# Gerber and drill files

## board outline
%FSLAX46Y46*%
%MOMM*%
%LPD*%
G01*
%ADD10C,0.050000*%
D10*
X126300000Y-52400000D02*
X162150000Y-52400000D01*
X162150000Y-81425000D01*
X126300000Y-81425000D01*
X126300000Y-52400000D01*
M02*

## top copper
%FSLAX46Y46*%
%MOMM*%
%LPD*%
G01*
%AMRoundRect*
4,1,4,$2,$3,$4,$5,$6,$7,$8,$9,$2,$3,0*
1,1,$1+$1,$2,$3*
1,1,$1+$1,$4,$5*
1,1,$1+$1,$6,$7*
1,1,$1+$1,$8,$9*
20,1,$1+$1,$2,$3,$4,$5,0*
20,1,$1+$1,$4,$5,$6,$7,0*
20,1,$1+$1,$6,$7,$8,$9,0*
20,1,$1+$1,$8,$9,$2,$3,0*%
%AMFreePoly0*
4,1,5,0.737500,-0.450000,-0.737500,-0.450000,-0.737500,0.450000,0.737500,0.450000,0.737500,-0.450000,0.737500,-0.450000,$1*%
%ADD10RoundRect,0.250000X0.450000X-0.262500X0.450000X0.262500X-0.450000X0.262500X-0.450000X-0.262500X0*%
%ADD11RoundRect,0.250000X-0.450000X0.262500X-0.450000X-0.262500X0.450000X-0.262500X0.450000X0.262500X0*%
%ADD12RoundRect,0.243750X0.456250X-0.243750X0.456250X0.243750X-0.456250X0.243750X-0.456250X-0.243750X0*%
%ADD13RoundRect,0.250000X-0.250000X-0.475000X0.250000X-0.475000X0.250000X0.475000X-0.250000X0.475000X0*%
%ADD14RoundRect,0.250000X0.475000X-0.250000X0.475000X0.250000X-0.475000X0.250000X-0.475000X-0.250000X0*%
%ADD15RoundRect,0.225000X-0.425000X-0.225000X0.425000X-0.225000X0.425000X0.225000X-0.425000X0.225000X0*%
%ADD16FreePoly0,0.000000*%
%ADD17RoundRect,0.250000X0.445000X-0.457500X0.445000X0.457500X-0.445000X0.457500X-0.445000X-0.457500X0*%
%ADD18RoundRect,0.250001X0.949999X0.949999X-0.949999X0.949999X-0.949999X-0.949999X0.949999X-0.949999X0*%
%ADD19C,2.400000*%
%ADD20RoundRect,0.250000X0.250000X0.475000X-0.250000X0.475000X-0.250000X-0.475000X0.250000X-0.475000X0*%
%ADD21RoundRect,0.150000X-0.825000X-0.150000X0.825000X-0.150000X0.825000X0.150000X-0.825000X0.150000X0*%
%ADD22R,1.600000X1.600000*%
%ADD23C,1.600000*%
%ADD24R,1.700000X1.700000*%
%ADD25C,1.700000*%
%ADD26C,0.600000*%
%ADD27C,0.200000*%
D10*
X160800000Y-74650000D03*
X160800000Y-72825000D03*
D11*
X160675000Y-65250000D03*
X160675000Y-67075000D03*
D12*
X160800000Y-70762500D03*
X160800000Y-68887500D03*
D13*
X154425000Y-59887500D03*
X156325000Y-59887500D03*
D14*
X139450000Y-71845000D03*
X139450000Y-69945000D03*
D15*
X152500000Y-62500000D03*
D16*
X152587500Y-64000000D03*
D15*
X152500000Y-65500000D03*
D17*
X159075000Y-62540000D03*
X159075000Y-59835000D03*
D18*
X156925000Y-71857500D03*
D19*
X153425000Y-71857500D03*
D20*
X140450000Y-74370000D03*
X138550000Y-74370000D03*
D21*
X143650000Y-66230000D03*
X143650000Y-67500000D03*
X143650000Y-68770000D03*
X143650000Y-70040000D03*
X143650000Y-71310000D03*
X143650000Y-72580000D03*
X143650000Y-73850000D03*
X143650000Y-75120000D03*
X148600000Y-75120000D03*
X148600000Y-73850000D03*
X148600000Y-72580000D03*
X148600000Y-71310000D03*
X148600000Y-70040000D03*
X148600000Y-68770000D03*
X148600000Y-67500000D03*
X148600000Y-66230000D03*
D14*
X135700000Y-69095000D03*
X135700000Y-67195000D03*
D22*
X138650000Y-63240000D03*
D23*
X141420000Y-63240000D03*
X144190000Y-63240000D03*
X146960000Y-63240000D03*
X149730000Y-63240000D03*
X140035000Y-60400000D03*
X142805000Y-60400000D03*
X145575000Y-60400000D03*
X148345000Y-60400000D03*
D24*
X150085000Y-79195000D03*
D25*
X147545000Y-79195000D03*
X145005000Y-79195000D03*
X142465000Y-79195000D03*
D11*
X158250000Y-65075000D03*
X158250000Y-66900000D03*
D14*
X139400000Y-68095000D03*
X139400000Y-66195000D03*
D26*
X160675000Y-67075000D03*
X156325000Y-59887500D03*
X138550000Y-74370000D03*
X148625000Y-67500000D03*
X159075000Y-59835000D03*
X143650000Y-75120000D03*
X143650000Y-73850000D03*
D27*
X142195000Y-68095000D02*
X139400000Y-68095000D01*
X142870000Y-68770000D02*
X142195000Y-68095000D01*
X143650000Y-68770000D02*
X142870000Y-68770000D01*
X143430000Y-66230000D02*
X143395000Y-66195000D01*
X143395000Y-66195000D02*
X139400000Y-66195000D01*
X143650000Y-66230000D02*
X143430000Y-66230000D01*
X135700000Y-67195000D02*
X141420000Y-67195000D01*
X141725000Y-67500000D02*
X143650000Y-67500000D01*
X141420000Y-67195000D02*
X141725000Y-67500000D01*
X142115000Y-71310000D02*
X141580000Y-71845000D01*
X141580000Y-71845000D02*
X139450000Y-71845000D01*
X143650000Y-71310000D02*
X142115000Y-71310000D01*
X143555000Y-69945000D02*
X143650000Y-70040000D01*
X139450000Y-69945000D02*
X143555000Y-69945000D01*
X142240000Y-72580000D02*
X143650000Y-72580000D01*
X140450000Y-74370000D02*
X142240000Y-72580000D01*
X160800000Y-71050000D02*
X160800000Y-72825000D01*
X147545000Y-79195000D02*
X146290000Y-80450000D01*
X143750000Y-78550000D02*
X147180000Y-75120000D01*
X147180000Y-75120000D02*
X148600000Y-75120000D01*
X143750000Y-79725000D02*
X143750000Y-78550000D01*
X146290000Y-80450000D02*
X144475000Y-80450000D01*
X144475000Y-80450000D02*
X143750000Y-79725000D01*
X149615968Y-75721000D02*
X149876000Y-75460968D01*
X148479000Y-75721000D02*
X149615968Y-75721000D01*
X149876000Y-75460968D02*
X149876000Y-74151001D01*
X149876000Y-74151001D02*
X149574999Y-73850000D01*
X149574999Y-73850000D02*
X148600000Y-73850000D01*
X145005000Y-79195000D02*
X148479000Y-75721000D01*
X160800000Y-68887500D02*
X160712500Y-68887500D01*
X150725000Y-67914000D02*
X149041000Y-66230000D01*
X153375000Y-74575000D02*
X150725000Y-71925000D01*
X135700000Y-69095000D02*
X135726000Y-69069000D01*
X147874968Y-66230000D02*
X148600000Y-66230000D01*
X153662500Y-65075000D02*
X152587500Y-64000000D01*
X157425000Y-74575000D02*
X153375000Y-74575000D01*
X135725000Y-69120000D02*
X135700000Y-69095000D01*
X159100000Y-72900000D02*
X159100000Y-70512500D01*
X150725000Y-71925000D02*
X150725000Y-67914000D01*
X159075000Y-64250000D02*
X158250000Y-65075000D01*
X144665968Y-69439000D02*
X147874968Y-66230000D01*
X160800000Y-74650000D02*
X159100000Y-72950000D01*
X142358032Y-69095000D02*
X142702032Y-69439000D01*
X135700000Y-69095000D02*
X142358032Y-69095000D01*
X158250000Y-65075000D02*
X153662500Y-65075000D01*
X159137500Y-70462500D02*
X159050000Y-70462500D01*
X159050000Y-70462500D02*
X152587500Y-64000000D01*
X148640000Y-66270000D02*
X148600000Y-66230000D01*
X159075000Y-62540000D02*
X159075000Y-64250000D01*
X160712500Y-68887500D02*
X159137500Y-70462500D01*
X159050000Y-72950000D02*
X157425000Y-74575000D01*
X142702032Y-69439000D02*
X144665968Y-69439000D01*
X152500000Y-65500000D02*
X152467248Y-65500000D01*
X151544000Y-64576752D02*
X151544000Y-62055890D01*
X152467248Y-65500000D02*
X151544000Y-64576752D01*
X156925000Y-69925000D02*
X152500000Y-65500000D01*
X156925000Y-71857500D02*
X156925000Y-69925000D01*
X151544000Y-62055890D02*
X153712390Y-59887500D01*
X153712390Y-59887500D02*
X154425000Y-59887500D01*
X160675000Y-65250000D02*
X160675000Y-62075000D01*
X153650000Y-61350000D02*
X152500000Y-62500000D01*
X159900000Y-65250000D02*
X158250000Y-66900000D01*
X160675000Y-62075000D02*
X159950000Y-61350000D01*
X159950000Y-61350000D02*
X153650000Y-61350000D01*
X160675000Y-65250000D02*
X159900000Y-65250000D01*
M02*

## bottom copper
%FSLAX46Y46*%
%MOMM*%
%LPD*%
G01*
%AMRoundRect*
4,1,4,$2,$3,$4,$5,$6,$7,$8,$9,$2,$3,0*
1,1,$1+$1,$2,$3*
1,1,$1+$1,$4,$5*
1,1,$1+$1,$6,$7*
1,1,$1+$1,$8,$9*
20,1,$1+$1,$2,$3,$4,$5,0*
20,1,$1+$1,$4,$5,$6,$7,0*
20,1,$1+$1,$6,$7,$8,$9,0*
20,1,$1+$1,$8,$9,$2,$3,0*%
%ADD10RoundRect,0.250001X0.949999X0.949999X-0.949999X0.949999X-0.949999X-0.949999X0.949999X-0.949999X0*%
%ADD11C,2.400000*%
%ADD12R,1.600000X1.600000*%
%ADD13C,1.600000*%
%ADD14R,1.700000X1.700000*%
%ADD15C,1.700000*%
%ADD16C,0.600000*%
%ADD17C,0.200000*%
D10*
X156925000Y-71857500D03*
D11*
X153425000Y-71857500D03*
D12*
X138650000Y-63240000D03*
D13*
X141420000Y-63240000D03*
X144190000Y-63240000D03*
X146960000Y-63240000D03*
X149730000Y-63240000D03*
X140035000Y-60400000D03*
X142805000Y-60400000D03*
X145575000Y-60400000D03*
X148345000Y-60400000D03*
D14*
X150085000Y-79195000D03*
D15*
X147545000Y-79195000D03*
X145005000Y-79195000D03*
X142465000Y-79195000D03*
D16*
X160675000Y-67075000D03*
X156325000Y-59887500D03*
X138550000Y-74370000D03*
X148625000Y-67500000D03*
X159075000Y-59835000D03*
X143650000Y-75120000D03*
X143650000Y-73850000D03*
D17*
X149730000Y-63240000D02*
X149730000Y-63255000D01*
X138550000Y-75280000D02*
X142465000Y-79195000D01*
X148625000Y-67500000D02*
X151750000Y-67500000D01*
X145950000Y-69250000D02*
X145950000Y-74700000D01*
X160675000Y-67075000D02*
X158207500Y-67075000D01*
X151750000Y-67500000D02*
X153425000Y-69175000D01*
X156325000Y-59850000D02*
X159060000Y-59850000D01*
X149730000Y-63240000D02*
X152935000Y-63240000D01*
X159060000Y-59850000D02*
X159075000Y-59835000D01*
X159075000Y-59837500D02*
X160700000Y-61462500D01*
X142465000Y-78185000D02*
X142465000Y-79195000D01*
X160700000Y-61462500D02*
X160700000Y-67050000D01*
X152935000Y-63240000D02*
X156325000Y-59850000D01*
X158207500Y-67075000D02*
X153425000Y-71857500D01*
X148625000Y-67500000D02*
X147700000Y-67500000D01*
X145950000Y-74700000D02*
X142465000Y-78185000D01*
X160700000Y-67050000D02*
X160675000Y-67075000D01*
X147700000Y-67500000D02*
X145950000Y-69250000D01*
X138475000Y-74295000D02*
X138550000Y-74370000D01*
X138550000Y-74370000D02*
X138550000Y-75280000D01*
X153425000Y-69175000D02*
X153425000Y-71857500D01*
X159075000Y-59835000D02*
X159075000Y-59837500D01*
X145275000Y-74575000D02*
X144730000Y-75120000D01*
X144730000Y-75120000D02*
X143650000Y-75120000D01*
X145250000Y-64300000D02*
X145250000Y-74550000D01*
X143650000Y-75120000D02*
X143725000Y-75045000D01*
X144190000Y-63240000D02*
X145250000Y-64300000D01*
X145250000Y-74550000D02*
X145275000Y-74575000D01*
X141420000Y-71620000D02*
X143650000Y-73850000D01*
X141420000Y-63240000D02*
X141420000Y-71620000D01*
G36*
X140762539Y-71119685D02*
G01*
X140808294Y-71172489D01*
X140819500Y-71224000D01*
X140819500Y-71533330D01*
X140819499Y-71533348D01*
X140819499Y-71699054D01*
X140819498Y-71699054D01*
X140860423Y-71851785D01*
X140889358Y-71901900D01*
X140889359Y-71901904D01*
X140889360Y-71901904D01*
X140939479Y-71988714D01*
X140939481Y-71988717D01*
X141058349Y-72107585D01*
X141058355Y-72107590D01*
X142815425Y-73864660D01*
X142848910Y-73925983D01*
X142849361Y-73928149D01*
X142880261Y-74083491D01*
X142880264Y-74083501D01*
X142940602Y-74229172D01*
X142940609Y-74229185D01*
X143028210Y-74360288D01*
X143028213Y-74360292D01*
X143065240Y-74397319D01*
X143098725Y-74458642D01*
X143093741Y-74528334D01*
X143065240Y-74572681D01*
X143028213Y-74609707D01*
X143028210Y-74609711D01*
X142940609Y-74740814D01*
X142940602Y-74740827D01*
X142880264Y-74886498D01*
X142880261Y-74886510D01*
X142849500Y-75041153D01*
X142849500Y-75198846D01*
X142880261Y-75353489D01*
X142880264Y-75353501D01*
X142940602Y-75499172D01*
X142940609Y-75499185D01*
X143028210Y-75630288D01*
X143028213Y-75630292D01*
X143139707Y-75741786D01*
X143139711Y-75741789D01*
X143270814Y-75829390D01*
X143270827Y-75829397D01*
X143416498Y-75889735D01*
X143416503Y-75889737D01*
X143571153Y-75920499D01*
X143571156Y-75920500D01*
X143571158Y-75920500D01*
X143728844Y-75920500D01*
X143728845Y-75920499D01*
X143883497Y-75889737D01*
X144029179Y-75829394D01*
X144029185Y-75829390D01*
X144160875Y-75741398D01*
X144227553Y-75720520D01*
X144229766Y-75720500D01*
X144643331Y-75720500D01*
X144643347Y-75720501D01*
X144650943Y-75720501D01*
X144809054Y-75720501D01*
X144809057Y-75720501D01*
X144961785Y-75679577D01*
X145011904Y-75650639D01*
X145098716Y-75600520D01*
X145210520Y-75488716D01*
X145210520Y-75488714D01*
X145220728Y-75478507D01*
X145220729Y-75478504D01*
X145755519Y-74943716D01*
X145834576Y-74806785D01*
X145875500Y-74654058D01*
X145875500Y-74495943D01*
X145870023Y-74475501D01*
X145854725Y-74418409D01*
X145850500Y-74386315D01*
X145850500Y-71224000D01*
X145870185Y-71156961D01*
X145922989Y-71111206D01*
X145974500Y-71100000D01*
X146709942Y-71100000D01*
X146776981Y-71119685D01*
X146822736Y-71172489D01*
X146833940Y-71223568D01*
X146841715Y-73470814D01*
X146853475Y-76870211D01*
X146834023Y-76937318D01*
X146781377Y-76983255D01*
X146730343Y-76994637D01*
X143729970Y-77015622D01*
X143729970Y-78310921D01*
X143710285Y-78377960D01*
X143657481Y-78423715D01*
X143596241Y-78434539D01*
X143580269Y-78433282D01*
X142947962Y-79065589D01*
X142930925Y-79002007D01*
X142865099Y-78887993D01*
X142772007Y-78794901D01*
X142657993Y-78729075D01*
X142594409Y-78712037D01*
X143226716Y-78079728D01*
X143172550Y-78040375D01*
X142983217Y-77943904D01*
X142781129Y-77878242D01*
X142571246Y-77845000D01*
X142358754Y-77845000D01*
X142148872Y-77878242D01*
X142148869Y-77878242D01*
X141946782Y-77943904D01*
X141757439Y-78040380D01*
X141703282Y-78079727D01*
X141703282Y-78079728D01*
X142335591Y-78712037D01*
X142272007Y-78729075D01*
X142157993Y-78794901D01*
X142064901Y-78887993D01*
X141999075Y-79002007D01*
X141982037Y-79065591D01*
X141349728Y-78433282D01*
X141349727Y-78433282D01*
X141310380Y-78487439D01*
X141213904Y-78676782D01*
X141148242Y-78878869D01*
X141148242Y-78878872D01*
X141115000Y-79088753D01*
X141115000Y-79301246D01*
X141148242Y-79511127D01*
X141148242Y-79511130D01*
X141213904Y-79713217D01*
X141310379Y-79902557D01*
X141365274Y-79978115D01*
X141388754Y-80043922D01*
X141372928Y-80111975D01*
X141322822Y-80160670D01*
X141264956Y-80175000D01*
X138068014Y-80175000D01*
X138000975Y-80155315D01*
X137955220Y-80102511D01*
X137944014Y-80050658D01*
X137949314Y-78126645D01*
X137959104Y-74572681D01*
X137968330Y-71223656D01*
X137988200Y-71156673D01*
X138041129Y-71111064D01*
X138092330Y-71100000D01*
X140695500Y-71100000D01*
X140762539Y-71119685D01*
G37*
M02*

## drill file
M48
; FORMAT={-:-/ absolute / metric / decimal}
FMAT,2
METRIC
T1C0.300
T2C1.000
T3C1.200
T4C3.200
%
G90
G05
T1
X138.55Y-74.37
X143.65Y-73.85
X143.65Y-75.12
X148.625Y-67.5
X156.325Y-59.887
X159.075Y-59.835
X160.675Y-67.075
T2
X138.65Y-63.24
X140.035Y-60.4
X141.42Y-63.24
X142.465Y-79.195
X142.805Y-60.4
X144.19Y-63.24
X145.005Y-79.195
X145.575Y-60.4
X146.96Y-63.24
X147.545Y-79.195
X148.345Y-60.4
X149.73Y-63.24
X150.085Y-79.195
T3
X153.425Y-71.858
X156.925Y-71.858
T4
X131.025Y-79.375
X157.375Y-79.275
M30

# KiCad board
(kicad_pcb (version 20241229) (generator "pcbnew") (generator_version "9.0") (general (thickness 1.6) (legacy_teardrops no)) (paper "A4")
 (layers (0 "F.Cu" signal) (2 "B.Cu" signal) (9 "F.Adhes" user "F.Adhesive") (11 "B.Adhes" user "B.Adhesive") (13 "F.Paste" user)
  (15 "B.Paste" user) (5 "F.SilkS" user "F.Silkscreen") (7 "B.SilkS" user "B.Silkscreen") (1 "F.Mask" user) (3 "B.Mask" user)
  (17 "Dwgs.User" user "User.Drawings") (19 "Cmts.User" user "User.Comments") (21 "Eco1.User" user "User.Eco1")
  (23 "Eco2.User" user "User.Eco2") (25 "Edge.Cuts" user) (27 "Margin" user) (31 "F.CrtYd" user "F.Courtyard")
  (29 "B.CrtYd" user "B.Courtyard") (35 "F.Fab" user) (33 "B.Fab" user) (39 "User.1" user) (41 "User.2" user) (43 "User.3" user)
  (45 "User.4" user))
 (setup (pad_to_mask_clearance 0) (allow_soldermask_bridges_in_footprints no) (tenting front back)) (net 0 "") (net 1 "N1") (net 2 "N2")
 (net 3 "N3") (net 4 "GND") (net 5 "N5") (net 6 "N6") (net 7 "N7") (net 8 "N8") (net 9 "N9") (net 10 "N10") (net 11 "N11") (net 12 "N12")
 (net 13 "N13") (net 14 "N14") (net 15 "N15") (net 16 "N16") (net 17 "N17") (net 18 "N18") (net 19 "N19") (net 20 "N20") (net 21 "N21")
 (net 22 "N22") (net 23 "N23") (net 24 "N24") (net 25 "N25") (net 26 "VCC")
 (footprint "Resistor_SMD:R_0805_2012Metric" (layer "F.Cu") (at 160.8 73.7375 90)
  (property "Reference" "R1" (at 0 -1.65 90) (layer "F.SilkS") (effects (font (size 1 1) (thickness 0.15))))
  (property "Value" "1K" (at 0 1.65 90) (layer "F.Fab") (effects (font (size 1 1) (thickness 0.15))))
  (pad "1" smd roundrect (at -0.9125 0 90) (size 1.025 1.4) (layers "F.Cu" "F.Mask" "F.Paste") (roundrect_rratio 0.243902) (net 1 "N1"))
  (pad "2" smd roundrect (at 0.9125 0 90) (size 1.025 1.4) (layers "F.Cu" "F.Mask" "F.Paste") (roundrect_rratio 0.243902) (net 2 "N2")))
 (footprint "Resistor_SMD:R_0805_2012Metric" (layer "F.Cu") (at 160.675 66.1625 -90)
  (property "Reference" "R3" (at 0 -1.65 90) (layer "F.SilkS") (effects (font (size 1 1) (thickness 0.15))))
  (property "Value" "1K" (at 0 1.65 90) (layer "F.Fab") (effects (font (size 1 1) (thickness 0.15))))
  (pad "1" smd roundrect (at -0.9125 0 270) (size 1.025 1.4) (layers "F.Cu" "F.Mask" "F.Paste") (roundrect_rratio 0.243902) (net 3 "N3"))
  (pad "2" smd roundrect (at 0.9125 0 270) (size 1.025 1.4) (layers "F.Cu" "F.Mask" "F.Paste") (roundrect_rratio 0.243902) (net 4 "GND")))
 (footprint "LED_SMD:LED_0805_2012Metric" (layer "F.Cu") (at 160.8 69.825 90)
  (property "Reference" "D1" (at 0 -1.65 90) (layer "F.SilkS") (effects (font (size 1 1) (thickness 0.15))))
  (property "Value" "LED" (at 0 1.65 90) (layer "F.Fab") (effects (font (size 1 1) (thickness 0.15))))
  (pad "1" smd roundrect (at -0.9375 0 90) (size 0.975 1.4) (layers "F.Cu" "F.Mask" "F.Paste") (roundrect_rratio 0.25) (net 2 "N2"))
  (pad "2" smd roundrect (at 0.9375 0 90) (size 0.975 1.4) (layers "F.Cu" "F.Mask" "F.Paste") (roundrect_rratio 0.25) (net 1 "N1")))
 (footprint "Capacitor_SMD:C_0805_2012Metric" (layer "F.Cu") (at 155.375 59.8875)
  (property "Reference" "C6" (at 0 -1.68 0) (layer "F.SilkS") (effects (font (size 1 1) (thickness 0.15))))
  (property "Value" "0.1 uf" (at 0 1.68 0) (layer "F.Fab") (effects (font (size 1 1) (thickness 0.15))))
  (pad "1" smd roundrect (at -0.95 0) (size 1 1.45) (layers "F.Cu" "F.Mask" "F.Paste") (roundrect_rratio 0.25) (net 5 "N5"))
  (pad "2" smd roundrect (at 0.95 0) (size 1 1.45) (layers "F.Cu" "F.Mask" "F.Paste") (roundrect_rratio 0.25) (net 4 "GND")))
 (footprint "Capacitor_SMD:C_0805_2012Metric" (layer "F.Cu") (at 139.45 70.895 90)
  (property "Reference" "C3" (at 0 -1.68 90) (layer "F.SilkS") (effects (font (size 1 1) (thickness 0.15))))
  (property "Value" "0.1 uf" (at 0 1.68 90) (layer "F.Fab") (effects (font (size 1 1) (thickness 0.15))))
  (pad "1" smd roundrect (at -0.95 0 90) (size 1 1.45) (layers "F.Cu" "F.Mask" "F.Paste") (roundrect_rratio 0.25) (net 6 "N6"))
  (pad "2" smd roundrect (at 0.95 0 90) (size 1 1.45) (layers "F.Cu" "F.Mask" "F.Paste") (roundrect_rratio 0.25) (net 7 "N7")))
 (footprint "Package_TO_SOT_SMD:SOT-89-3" (layer "F.Cu") (at 154.45 64)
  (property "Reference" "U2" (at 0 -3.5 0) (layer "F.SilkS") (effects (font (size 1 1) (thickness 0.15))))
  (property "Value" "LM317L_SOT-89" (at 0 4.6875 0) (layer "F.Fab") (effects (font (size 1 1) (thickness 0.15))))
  (pad "1" smd roundrect (at -1.95 -1.5) (size 1.3 0.9) (layers "F.Cu" "F.Mask" "F.Paste") (roundrect_rratio 0.25) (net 3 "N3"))
  (pad "2" smd custom (at -1.8625 0) (size 1.475 0.9) (layers "F.Cu" "F.Mask" "F.Paste") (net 1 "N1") (zone_connect 2)
   (thermal_bridge_angle 45) (options (clearance outline) (anchor rect)) (primitives))
  (pad "3" smd roundrect (at -1.95 1.5) (size 1.3 0.9) (layers "F.Cu" "F.Mask" "F.Paste") (roundrect_rratio 0.25) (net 5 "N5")))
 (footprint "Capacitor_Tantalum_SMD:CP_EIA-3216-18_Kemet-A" (layer "F.Cu") (at 159.075 61.1875 90)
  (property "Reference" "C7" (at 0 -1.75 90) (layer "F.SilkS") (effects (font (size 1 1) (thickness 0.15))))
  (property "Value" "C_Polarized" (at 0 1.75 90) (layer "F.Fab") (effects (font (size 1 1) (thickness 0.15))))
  (pad "1" smd roundrect (at -1.3525 0 90) (size 1.415 1.39) (layers "F.Cu" "F.Mask" "F.Paste") (roundrect_rratio 0.179856) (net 1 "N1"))
  (pad "2" smd roundrect (at 1.3525 0 90) (size 1.415 1.39) (layers "F.Cu" "F.Mask" "F.Paste") (roundrect_rratio 0.179856) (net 4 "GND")))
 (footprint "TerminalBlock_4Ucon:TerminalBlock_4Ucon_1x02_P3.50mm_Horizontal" (layer "F.Cu") (at 156.925 71.8575 180)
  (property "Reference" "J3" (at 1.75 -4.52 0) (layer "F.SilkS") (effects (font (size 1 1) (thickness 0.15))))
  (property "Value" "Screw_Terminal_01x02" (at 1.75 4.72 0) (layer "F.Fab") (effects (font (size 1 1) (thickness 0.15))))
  (pad "1" thru_hole roundrect (at 0 0 180) (size 2.4 2.4) (drill 1.2) (layers "*.Cu" "*.Mask") (remove_unused_layers no)
   (roundrect_rratio 0.104167) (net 5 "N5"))
  (pad "2" thru_hole circle (at 3.5 0 180) (size 2.4 2.4) (drill 1.2) (layers "*.Cu" "*.Mask") (remove_unused_layers no) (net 4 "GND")))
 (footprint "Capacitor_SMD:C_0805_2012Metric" (layer "F.Cu") (at 139.5 74.37 180)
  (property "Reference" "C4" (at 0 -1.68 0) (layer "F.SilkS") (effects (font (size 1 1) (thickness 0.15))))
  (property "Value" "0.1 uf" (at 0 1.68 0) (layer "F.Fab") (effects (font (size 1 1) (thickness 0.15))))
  (pad "1" smd roundrect (at -0.95 0 180) (size 1 1.45) (layers "F.Cu" "F.Mask" "F.Paste") (roundrect_rratio 0.25) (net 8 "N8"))
  (pad "2" smd roundrect (at 0.95 0 180) (size 1 1.45) (layers "F.Cu" "F.Mask" "F.Paste") (roundrect_rratio 0.25) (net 4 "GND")))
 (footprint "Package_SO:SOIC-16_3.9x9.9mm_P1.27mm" (layer "F.Cu") (at 146.125 70.675)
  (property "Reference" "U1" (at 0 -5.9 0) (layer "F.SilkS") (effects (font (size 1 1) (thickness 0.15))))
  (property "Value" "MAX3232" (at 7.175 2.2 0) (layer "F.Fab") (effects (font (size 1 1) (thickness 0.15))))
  (pad "1" smd roundrect (at -2.475 -4.445) (size 1.95 0.6) (layers "F.Cu" "F.Mask" "F.Paste") (roundrect_rratio 0.25) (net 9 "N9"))
  (pad "2" smd roundrect (at -2.475 -3.175) (size 1.95 0.6) (layers "F.Cu" "F.Mask" "F.Paste") (roundrect_rratio 0.25) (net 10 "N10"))
  (pad "3" smd roundrect (at -2.475 -1.905) (size 1.95 0.6) (layers "F.Cu" "F.Mask" "F.Paste") (roundrect_rratio 0.25) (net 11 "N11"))
  (pad "4" smd roundrect (at -2.475 -0.635) (size 1.95 0.6) (layers "F.Cu" "F.Mask" "F.Paste") (roundrect_rratio 0.25) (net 7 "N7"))
  (pad "5" smd roundrect (at -2.475 0.635) (size 1.95 0.6) (layers "F.Cu" "F.Mask" "F.Paste") (roundrect_rratio 0.25) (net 6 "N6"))
  (pad "6" smd roundrect (at -2.475 1.905) (size 1.95 0.6) (layers "F.Cu" "F.Mask" "F.Paste") (roundrect_rratio 0.25) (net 8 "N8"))
  (pad "7" smd roundrect (at -2.475 3.175) (size 1.95 0.6) (layers "F.Cu" "F.Mask" "F.Paste") (roundrect_rratio 0.25) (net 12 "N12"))
  (pad "8" smd roundrect (at -2.475 4.445) (size 1.95 0.6) (layers "F.Cu" "F.Mask" "F.Paste") (roundrect_rratio 0.25) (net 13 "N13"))
  (pad "9" smd roundrect (at 2.475 4.445) (size 1.95 0.6) (layers "F.Cu" "F.Mask" "F.Paste") (roundrect_rratio 0.25) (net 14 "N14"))
  (pad "10" smd roundrect (at 2.475 3.175) (size 1.95 0.6) (layers "F.Cu" "F.Mask" "F.Paste") (roundrect_rratio 0.25) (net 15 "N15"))
  (pad "11" smd roundrect (at 2.475 1.905) (size 1.95 0.6) (layers "F.Cu" "F.Mask" "F.Paste") (roundrect_rratio 0.25) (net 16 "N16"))
  (pad "12" smd roundrect (at 2.475 0.635) (size 1.95 0.6) (layers "F.Cu" "F.Mask" "F.Paste") (roundrect_rratio 0.25) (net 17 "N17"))
  (pad "13" smd roundrect (at 2.475 -0.635) (size 1.95 0.6) (layers "F.Cu" "F.Mask" "F.Paste") (roundrect_rratio 0.25) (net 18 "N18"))
  (pad "14" smd roundrect (at 2.475 -1.905) (size 1.95 0.6) (layers "F.Cu" "F.Mask" "F.Paste") (roundrect_rratio 0.25) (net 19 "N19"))
  (pad "15" smd roundrect (at 2.475 -3.175) (size 1.95 0.6) (layers "F.Cu" "F.Mask" "F.Paste") (roundrect_rratio 0.25) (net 4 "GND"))
  (pad "16" smd roundrect (at 2.475 -4.445) (size 1.95 0.6) (layers "F.Cu" "F.Mask" "F.Paste") (roundrect_rratio 0.25) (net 1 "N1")))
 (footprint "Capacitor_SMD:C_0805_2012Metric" (layer "F.Cu") (at 135.7 68.145 90)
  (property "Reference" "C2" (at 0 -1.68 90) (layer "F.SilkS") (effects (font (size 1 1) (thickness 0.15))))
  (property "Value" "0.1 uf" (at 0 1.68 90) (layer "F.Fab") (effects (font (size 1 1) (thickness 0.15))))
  (pad "1" smd roundrect (at -0.95 0 90) (size 1 1.45) (layers "F.Cu" "F.Mask" "F.Paste") (roundrect_rratio 0.25) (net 1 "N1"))
  (pad "2" smd roundrect (at 0.95 0 90) (size 1 1.45) (layers "F.Cu" "F.Mask" "F.Paste") (roundrect_rratio 0.25) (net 10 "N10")))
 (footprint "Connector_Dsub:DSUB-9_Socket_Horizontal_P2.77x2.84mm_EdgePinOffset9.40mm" (layer "F.Cu") (at 138.65 63.24 180)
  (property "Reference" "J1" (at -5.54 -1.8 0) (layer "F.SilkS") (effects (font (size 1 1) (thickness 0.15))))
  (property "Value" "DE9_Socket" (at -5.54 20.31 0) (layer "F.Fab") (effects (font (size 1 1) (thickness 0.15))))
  (pad "1" thru_hole rect (at 0 0 180) (size 1.6 1.6) (drill 1) (layers "*.Cu" "*.Mask") (remove_unused_layers no) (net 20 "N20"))
  (pad "2" thru_hole circle (at -2.77 0 180) (size 1.6 1.6) (drill 1) (layers "*.Cu" "*.Mask") (remove_unused_layers no) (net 12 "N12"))
  (pad "3" thru_hole circle (at -5.54 0 180) (size 1.6 1.6) (drill 1) (layers "*.Cu" "*.Mask") (remove_unused_layers no) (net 13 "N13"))
  (pad "4" thru_hole circle (at -8.31 0 180) (size 1.6 1.6) (drill 1) (layers "*.Cu" "*.Mask") (remove_unused_layers no) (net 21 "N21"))
  (pad "5" thru_hole circle (at -11.08 0 180) (size 1.6 1.6) (drill 1) (layers "*.Cu" "*.Mask") (remove_unused_layers no) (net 4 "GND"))
  (pad "6" thru_hole circle (at -1.385 2.84 180) (size 1.6 1.6) (drill 1) (layers "*.Cu" "*.Mask") (remove_unused_layers no) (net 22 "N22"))
  (pad "7" thru_hole circle (at -4.155 2.84 180) (size 1.6 1.6) (drill 1) (layers "*.Cu" "*.Mask") (remove_unused_layers no) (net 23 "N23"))
  (pad "8" thru_hole circle (at -6.925 2.84 180) (size 1.6 1.6) (drill 1) (layers "*.Cu" "*.Mask") (remove_unused_layers no) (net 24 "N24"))
  (pad "9" thru_hole circle (at -9.695 2.84 180) (size 1.6 1.6) (drill 1) (layers "*.Cu" "*.Mask") (remove_unused_layers no) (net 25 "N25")))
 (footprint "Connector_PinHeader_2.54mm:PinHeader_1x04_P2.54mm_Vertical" (layer "F.Cu") (at 150.085 79.195 -90)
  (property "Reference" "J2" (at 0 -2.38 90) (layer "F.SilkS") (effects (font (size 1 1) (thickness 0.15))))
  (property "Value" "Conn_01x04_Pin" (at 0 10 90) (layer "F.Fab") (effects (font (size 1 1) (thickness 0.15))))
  (pad "1" thru_hole rect (at 0 0 270) (size 1.7 1.7) (drill 1) (layers "*.Cu" "*.Mask") (remove_unused_layers no) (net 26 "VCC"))
  (pad "2" thru_hole circle (at 0 2.54 270) (size 1.7 1.7) (drill 1) (layers "*.Cu" "*.Mask") (remove_unused_layers no) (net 14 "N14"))
  (pad "3" thru_hole circle (at 0 5.08 270) (size 1.7 1.7) (drill 1) (layers "*.Cu" "*.Mask") (remove_unused_layers no) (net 15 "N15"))
  (pad "4" thru_hole circle (at 0 7.62 270) (size 1.7 1.7) (drill 1) (layers "*.Cu" "*.Mask") (remove_unused_layers no) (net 4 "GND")))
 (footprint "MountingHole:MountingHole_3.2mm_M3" (layer "F.Cu") (at 157.375 79.275)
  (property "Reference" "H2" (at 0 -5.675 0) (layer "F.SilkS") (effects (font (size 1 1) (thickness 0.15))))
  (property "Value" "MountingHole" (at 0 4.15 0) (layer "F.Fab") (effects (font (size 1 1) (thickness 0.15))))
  (pad "" np_thru_hole circle (at 0 0) (size 3.2 3.2) (drill 3.2) (layers "*.Cu" "*.Mask")))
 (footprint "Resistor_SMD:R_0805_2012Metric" (layer "F.Cu") (at 158.25 65.9875 -90)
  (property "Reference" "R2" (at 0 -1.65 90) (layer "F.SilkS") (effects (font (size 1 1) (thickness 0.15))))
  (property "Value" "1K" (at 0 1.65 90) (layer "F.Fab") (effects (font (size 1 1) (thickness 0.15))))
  (pad "1" smd roundrect (at -0.9125 0 270) (size 1.025 1.4) (layers "F.Cu" "F.Mask" "F.Paste") (roundrect_rratio 0.243902) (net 1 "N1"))
  (pad "2" smd roundrect (at 0.9125 0 270) (size 1.025 1.4) (layers "F.Cu" "F.Mask" "F.Paste") (roundrect_rratio 0.243902) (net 3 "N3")))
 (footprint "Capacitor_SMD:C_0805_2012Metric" (layer "F.Cu") (at 139.4 67.145 90)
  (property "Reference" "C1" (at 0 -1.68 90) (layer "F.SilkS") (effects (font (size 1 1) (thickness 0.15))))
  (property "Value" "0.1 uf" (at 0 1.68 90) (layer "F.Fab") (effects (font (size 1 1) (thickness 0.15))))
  (pad "1" smd roundrect (at -0.95 0 90) (size 1 1.45) (layers "F.Cu" "F.Mask" "F.Paste") (roundrect_rratio 0.25) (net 11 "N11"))
  (pad "2" smd roundrect (at 0.95 0 90) (size 1 1.45) (layers "F.Cu" "F.Mask" "F.Paste") (roundrect_rratio 0.25) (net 9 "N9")))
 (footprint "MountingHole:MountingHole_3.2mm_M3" (layer "F.Cu") (at 131.025 79.375)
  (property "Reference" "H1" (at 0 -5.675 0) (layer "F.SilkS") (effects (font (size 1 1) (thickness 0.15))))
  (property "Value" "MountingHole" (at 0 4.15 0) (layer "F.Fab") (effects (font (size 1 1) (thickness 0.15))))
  (pad "" np_thru_hole circle (at 0 0) (size 3.2 3.2) (drill 3.2) (layers "*.Cu" "*.Mask")))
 (gr_rect (start 126.3 52.4) (end 162.15 81.425) (stroke (width 0.05) (type solid)) (fill no) (layer "Edge.Cuts"))
 (segment (start 142.195 68.095) (end 139.4 68.095) (width 0.2) (layer "F.Cu") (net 11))
 (segment (start 142.87 68.77) (end 142.195 68.095) (width 0.2) (layer "F.Cu") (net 11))
 (segment (start 143.65 68.77) (end 142.87 68.77) (width 0.2) (layer "F.Cu") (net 11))
 (segment (start 143.43 66.23) (end 143.395 66.195) (width 0.2) (layer "F.Cu") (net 9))
 (segment (start 143.395 66.195) (end 139.4 66.195) (width 0.2) (layer "F.Cu") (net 9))
 (segment (start 143.65 66.23) (end 143.43 66.23) (width 0.2) (layer "F.Cu") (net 9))
 (segment (start 135.7 67.195) (end 141.42 67.195) (width 0.2) (layer "F.Cu") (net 10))
 (segment (start 141.725 67.5) (end 143.65 67.5) (width 0.2) (layer "F.Cu") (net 10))
 (segment (start 141.42 67.195) (end 141.725 67.5) (width 0.2) (layer "F.Cu") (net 10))
 (segment (start 142.115 71.31) (end 141.58 71.845) (width 0.2) (layer "F.Cu") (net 6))
 (segment (start 141.58 71.845) (end 139.45 71.845) (width 0.2) (layer "F.Cu") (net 6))
 (segment (start 143.65 71.31) (end 142.115 71.31) (width 0.2) (layer "F.Cu") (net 6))
 (segment (start 143.555 69.945) (end 143.65 70.04) (width 0.2) (layer "F.Cu") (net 7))
 (segment (start 139.45 69.945) (end 143.555 69.945) (width 0.2) (layer "F.Cu") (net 7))
 (via (at 160.675 67.075) (size 0.6) (drill 0.3) (layers "F.Cu" "B.Cu") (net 4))
 (via (at 156.325 59.8875) (size 0.6) (drill 0.3) (layers "F.Cu" "B.Cu") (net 4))
 (via (at 138.55 74.37) (size 0.6) (drill 0.3) (layers "F.Cu" "B.Cu") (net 4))
 (via (at 148.625 67.5) (size 0.6) (drill 0.3) (layers "F.Cu" "B.Cu") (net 4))
 (via (at 159.075 59.835) (size 0.6) (drill 0.3) (layers "F.Cu" "B.Cu") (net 4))
 (segment (start 149.73 63.24) (end 149.73 63.255) (width 0.2) (layer "B.Cu") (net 4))
 (segment (start 138.55 75.28) (end 142.465 79.195) (width 0.2) (layer "B.Cu") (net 4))
 (segment (start 148.625 67.5) (end 151.75 67.5) (width 0.2) (layer "B.Cu") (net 4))
 (segment (start 145.95 69.25) (end 145.95 74.7) (width 0.2) (layer "B.Cu") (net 4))
 (segment (start 160.675 67.075) (end 158.2075 67.075) (width 0.2) (layer "B.Cu") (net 4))
 (segment (start 151.75 67.5) (end 153.425 69.175) (width 0.2) (layer "B.Cu") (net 4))
 (segment (start 156.325 59.85) (end 159.06 59.85) (width 0.2) (layer "B.Cu") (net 4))
 (segment (start 149.73 63.24) (end 152.935 63.24) (width 0.2) (layer "B.Cu") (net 4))
 (segment (start 159.06 59.85) (end 159.075 59.835) (width 0.2) (layer "B.Cu") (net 4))
 (segment (start 159.075 59.8375) (end 160.7 61.4625) (width 0.2) (layer "B.Cu") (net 4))
 (segment (start 142.465 78.185) (end 142.465 79.195) (width 0.2) (layer "B.Cu") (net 4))
 (segment (start 160.7 61.4625) (end 160.7 67.05) (width 0.2) (layer "B.Cu") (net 4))
 (segment (start 152.935 63.24) (end 156.325 59.85) (width 0.2) (layer "B.Cu") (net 4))
 (segment (start 158.2075 67.075) (end 153.425 71.8575) (width 0.2) (layer "B.Cu") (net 4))
 (segment (start 148.625 67.5) (end 147.7 67.5) (width 0.2) (layer "B.Cu") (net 4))
 (segment (start 145.95 74.7) (end 142.465 78.185) (width 0.2) (layer "B.Cu") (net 4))
 (segment (start 160.7 67.05) (end 160.675 67.075) (width 0.2) (layer "B.Cu") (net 4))
 (segment (start 147.7 67.5) (end 145.95 69.25) (width 0.2) (layer "B.Cu") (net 4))
 (segment (start 138.475 74.295) (end 138.55 74.37) (width 0.2) (layer "B.Cu") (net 4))
 (segment (start 138.55 74.37) (end 138.55 75.28) (width 0.2) (layer "B.Cu") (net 4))
 (segment (start 153.425 69.175) (end 153.425 71.8575) (width 0.2) (layer "B.Cu") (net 4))
 (segment (start 159.075 59.835) (end 159.075 59.8375) (width 0.2) (layer "B.Cu") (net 4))
 (segment (start 142.24 72.58) (end 143.65 72.58) (width 0.2) (layer "F.Cu") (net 8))
 (segment (start 140.45 74.37) (end 142.24 72.58) (width 0.2) (layer "F.Cu") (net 8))
 (segment (start 160.8 71.05) (end 160.8 72.825) (width 0.2) (layer "F.Cu") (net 2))
 (via (at 143.65 75.12) (size 0.6) (drill 0.3) (layers "F.Cu" "B.Cu") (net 13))
 (segment (start 145.275 74.575) (end 144.73 75.12) (width 0.2) (layer "B.Cu") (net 13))
 (segment (start 144.73 75.12) (end 143.65 75.12) (width 0.2) (layer "B.Cu") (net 13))
 (segment (start 145.25 64.3) (end 145.25 74.55) (width 0.2) (layer "B.Cu") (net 13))
 (segment (start 143.65 75.12) (end 143.725 75.045) (width 0.2) (layer "B.Cu") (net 13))
 (segment (start 144.19 63.24) (end 145.25 64.3) (width 0.2) (layer "B.Cu") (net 13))
 (segment (start 145.25 74.55) (end 145.275 74.575) (width 0.2) (layer "B.Cu") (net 13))
 (via (at 143.65 73.85) (size 0.6) (drill 0.3) (layers "F.Cu" "B.Cu") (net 12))
 (segment (start 141.42 71.62) (end 143.65 73.85) (width 0.2) (layer "B.Cu") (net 12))
 (segment (start 141.42 63.24) (end 141.42 71.62) (width 0.2) (layer "B.Cu") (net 12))
 (segment (start 147.545 79.195) (end 146.29 80.45) (width 0.2) (layer "F.Cu") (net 14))
 (segment (start 143.75 78.55) (end 147.18 75.12) (width 0.2) (layer "F.Cu") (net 14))
 (segment (start 147.18 75.12) (end 148.6 75.12) (width 0.2) (layer "F.Cu") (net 14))
 (segment (start 143.75 79.725) (end 143.75 78.55) (width 0.2) (layer "F.Cu") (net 14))
 (segment (start 146.29 80.45) (end 144.475 80.45) (width 0.2) (layer "F.Cu") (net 14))
 (segment (start 144.475 80.45) (end 143.75 79.725) (width 0.2) (layer "F.Cu") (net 14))
 (segment (start 149.615968 75.721) (end 149.876 75.460968) (width 0.2) (layer "F.Cu") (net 15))
 (segment (start 148.479 75.721) (end 149.615968 75.721) (width 0.2) (layer "F.Cu") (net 15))
 (segment (start 149.876 75.460968) (end 149.876 74.151001) (width 0.2) (layer "F.Cu") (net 15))
 (segment (start 149.876 74.151001) (end 149.574999 73.85) (width 0.2) (layer "F.Cu") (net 15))
 (segment (start 149.574999 73.85) (end 148.6 73.85) (width 0.2) (layer "F.Cu") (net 15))
 (segment (start 145.005 79.195) (end 148.479 75.721) (width 0.2) (layer "F.Cu") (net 15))
 (segment (start 160.8 68.8875) (end 160.7125 68.8875) (width 0.2) (layer "F.Cu") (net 1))
 (segment (start 150.725 67.914) (end 149.041 66.23) (width 0.2) (layer "F.Cu") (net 1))
 (segment (start 153.375 74.575) (end 150.725 71.925) (width 0.2) (layer "F.Cu") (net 1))
 (segment (start 135.7 69.095) (end 135.726 69.069) (width 0.2) (layer "F.Cu") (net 1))
 (segment (start 147.874968 66.23) (end 148.6 66.23) (width 0.2) (layer "F.Cu") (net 1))
 (segment (start 153.6625 65.075) (end 152.5875 64) (width 0.2) (layer "F.Cu") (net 1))
 (segment (start 157.425 74.575) (end 153.375 74.575) (width 0.2) (layer "F.Cu") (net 1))
 (segment (start 135.725 69.12) (end 135.7 69.095) (width 0.2) (layer "F.Cu") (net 1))
 (segment (start 159.1 72.9) (end 159.1 70.5125) (width 0.2) (layer "F.Cu") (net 1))
 (segment (start 150.725 71.925) (end 150.725 67.914) (width 0.2) (layer "F.Cu") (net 1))
 (segment (start 159.075 64.25) (end 158.25 65.075) (width 0.2) (layer "F.Cu") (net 1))
 (segment (start 144.665968 69.439) (end 147.874968 66.23) (width 0.2) (layer "F.Cu") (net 1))
 (segment (start 160.8 74.65) (end 159.1 72.95) (width 0.2) (layer "F.Cu") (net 1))
 (segment (start 142.358032 69.095) (end 142.702032 69.439) (width 0.2) (layer "F.Cu") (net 1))
 (segment (start 135.7 69.095) (end 142.358032 69.095) (width 0.2) (layer "F.Cu") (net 1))
 (segment (start 158.25 65.075) (end 153.6625 65.075) (width 0.2) (layer "F.Cu") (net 1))
 (segment (start 159.1375 70.4625) (end 159.05 70.4625) (width 0.2) (layer "F.Cu") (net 1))
 (segment (start 159.05 70.4625) (end 152.5875 64) (width 0.2) (layer "F.Cu") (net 1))
 (segment (start 148.64 66.27) (end 148.6 66.23) (width 0.2) (layer "F.Cu") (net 1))
 (segment (start 159.075 62.54) (end 159.075 64.25) (width 0.2) (layer "F.Cu") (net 1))
 (segment (start 160.7125 68.8875) (end 159.1375 70.4625) (width 0.2) (layer "F.Cu") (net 1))
 (segment (start 159.05 72.95) (end 157.425 74.575) (width 0.2) (layer "F.Cu") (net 1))
 (segment (start 142.702032 69.439) (end 144.665968 69.439) (width 0.2) (layer "F.Cu") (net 1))
 (segment (start 152.5 65.5) (end 152.467248 65.5) (width 0.2) (layer "F.Cu") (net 5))
 (segment (start 151.544 64.576752) (end 151.544 62.05589) (width 0.2) (layer "F.Cu") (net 5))
 (segment (start 152.467248 65.5) (end 151.544 64.576752) (width 0.2) (layer "F.Cu") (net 5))
 (segment (start 156.925 69.925) (end 152.5 65.5) (width 0.2) (layer "F.Cu") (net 5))
 (segment (start 156.925 71.8575) (end 156.925 69.925) (width 0.2) (layer "F.Cu") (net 5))
 (segment (start 151.544 62.05589) (end 153.71239 59.8875) (width 0.2) (layer "F.Cu") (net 5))
 (segment (start 153.71239 59.8875) (end 154.425 59.8875) (width 0.2) (layer "F.Cu") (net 5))
 (segment (start 160.675 65.25) (end 160.675 62.075) (width 0.2) (layer "F.Cu") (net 3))
 (segment (start 153.65 61.35) (end 152.5 62.5) (width 0.2) (layer "F.Cu") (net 3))
 (segment (start 159.9 65.25) (end 158.25 66.9) (width 0.2) (layer "F.Cu") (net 3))
 (segment (start 160.675 62.075) (end 159.95 61.35) (width 0.2) (layer "F.Cu") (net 3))
 (segment (start 159.95 61.35) (end 153.65 61.35) (width 0.2) (layer "F.Cu") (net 3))
 (segment (start 160.675 65.25) (end 159.9 65.25) (width 0.2) (layer "F.Cu") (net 3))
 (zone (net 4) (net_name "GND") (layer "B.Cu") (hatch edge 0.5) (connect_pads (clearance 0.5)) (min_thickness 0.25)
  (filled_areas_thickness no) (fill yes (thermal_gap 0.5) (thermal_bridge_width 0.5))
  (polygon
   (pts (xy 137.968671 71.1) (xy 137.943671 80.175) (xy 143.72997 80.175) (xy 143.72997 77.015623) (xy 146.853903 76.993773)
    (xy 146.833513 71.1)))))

